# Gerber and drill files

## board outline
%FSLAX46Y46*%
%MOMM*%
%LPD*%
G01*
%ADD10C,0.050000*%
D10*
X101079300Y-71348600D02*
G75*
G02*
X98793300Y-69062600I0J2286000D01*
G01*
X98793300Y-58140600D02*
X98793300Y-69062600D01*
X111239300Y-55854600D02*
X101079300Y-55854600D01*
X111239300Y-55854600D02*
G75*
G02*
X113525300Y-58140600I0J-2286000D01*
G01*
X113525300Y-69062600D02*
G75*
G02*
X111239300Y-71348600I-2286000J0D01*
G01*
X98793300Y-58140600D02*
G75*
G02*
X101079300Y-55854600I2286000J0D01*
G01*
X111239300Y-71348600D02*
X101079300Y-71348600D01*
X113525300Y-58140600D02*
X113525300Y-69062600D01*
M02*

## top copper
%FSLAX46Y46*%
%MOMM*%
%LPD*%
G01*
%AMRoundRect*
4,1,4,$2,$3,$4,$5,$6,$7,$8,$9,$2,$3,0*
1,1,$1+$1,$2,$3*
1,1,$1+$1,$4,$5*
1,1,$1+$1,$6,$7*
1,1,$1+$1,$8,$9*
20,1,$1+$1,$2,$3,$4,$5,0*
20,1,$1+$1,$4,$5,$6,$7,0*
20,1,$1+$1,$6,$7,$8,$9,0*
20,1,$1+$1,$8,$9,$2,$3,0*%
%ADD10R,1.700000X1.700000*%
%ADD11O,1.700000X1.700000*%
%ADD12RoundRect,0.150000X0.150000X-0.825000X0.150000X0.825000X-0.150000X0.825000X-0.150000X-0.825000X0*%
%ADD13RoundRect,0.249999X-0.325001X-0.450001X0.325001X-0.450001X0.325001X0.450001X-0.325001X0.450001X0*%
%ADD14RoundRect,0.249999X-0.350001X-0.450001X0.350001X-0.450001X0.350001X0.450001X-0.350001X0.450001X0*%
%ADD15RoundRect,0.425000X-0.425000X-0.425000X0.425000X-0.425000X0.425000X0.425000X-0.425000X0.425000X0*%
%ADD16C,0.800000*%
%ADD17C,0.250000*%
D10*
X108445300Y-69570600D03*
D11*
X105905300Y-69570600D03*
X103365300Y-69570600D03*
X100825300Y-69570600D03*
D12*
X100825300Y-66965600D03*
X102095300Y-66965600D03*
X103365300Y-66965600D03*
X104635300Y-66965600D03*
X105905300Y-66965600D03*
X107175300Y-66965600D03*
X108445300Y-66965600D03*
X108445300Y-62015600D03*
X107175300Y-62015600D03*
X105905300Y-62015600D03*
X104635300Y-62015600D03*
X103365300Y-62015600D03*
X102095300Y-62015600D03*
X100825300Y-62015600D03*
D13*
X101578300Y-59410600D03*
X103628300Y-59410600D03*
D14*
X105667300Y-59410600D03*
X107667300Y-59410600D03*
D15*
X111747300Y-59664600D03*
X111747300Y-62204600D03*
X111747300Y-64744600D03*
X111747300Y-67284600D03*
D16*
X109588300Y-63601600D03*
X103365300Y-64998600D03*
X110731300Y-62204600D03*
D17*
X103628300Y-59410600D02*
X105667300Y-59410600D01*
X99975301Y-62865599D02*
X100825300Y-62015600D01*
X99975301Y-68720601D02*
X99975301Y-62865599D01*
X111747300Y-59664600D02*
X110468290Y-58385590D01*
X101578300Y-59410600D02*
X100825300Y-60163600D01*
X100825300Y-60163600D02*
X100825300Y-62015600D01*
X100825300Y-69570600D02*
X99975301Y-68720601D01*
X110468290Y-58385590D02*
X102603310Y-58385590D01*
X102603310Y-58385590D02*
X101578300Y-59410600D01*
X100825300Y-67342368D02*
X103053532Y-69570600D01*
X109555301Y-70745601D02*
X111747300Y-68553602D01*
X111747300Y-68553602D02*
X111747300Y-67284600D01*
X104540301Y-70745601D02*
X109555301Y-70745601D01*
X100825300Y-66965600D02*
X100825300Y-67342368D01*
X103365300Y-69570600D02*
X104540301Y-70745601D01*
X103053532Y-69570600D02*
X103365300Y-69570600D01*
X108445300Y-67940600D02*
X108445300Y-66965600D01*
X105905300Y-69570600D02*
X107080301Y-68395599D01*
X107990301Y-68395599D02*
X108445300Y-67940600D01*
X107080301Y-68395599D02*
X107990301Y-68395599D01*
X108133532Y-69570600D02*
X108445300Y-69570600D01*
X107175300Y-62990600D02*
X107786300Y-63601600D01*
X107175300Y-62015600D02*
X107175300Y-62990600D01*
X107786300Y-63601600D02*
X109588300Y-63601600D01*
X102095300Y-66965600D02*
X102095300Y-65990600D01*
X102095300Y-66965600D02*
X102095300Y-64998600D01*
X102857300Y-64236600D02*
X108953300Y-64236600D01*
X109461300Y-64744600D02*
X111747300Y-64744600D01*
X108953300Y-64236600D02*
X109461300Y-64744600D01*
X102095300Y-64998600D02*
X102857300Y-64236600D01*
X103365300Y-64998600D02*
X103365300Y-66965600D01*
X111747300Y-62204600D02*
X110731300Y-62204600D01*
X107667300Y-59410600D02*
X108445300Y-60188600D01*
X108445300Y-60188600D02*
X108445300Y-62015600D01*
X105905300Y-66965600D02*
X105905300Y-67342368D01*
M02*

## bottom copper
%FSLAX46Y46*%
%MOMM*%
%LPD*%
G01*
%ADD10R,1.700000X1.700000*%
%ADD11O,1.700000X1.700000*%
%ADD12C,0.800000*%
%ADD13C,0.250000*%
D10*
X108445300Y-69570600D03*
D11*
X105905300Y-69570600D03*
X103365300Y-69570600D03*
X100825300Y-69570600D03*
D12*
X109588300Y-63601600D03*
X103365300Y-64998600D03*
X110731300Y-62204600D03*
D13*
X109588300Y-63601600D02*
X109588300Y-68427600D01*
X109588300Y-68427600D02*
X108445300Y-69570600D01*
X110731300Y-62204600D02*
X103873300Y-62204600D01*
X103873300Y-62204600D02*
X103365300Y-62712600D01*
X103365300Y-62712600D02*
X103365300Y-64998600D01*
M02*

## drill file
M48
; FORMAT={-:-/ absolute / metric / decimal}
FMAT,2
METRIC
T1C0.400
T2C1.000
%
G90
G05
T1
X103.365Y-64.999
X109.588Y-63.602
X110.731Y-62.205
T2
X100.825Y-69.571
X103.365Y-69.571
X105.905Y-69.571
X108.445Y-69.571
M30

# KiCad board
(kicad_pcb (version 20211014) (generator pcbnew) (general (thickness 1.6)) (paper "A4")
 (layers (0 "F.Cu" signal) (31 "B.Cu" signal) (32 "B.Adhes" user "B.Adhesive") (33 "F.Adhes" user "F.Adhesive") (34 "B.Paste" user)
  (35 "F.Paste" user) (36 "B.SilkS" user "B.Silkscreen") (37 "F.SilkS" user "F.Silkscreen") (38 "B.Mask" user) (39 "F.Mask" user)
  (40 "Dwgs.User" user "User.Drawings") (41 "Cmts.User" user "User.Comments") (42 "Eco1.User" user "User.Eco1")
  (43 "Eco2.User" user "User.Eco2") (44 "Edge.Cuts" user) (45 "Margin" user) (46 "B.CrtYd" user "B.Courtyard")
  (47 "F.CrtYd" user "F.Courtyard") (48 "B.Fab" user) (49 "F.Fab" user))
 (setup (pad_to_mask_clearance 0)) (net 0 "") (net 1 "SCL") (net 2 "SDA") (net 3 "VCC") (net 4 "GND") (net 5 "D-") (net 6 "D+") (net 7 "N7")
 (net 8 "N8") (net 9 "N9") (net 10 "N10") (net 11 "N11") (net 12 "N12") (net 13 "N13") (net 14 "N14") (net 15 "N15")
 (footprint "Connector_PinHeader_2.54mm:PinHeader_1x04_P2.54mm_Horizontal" (layer "F.Cu") (at 108.4453 69.5706 -90)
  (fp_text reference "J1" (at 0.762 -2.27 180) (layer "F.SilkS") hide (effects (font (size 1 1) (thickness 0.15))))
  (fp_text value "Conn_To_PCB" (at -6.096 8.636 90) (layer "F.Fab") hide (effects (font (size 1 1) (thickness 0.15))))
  (pad "1" thru_hole rect locked (at 0 0 270) (size 1.7 1.7) (drill 1) (layers *.Cu *.Mask) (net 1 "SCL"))
  (pad "2" thru_hole oval locked (at 0 2.54 270) (size 1.7 1.7) (drill 1) (layers *.Cu *.Mask) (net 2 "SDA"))
  (pad "3" thru_hole oval locked (at 0 5.08 270) (size 1.7 1.7) (drill 1) (layers *.Cu *.Mask) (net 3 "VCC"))
  (pad "4" thru_hole oval locked (at 0 7.62 270) (size 1.7 1.7) (drill 1) (layers *.Cu *.Mask) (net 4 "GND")))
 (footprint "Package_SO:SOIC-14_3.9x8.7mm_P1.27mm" (layer "F.Cu") (at 104.6353 64.4906 90)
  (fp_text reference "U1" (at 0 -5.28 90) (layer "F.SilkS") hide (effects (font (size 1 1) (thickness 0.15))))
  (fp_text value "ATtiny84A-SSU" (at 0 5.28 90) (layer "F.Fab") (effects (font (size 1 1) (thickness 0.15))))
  (pad "1" smd roundrect locked (at -2.475 -3.81 90) (size 1.95 0.6) (layers "F.Cu" "F.Paste" "F.Mask") (roundrect_rratio 0.25)
   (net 3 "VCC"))
  (pad "2" smd roundrect locked (at -2.475 -2.54 90) (size 1.95 0.6) (layers "F.Cu" "F.Paste" "F.Mask") (roundrect_rratio 0.25) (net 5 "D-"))
  (pad "3" smd roundrect locked (at -2.475 -1.27 90) (size 1.95 0.6) (layers "F.Cu" "F.Paste" "F.Mask") (roundrect_rratio 0.25) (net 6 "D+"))
  (pad "4" smd roundrect locked (at -2.475 0 90) (size 1.95 0.6) (layers "F.Cu" "F.Paste" "F.Mask") (roundrect_rratio 0.25) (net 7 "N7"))
  (pad "5" smd roundrect locked (at -2.475 1.27 90) (size 1.95 0.6) (layers "F.Cu" "F.Paste" "F.Mask") (roundrect_rratio 0.25) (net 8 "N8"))
  (pad "6" smd roundrect locked (at -2.475 2.54 90) (size 1.95 0.6) (layers "F.Cu" "F.Paste" "F.Mask") (roundrect_rratio 0.25) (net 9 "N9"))
  (pad "7" smd roundrect locked (at -2.475 3.81 90) (size 1.95 0.6) (layers "F.Cu" "F.Paste" "F.Mask") (roundrect_rratio 0.25) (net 2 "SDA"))
  (pad "8" smd roundrect locked (at 2.475 3.81 90) (size 1.95 0.6) (layers "F.Cu" "F.Paste" "F.Mask") (roundrect_rratio 0.25) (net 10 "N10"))
  (pad "9" smd roundrect locked (at 2.475 2.54 90) (size 1.95 0.6) (layers "F.Cu" "F.Paste" "F.Mask") (roundrect_rratio 0.25) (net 1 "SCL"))
  (pad "10" smd roundrect locked (at 2.475 1.27 90) (size 1.95 0.6) (layers "F.Cu" "F.Paste" "F.Mask") (roundrect_rratio 0.25)
   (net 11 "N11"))
  (pad "11" smd roundrect locked (at 2.475 0 90) (size 1.95 0.6) (layers "F.Cu" "F.Paste" "F.Mask") (roundrect_rratio 0.25) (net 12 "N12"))
  (pad "12" smd roundrect locked (at 2.475 -1.27 90) (size 1.95 0.6) (layers "F.Cu" "F.Paste" "F.Mask") (roundrect_rratio 0.25)
   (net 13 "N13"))
  (pad "13" smd roundrect locked (at 2.475 -2.54 90) (size 1.95 0.6) (layers "F.Cu" "F.Paste" "F.Mask") (roundrect_rratio 0.25)
   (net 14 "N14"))
  (pad "14" smd roundrect locked (at 2.475 -3.81 90) (size 1.95 0.6) (layers "F.Cu" "F.Paste" "F.Mask") (roundrect_rratio 0.25)
   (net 4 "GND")))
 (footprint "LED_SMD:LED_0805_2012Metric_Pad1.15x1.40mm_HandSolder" (layer "F.Cu") (at 102.6033 59.4106)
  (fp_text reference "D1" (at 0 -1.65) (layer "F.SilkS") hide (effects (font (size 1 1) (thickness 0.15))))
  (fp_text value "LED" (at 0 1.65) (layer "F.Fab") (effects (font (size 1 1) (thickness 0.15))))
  (pad "1" smd roundrect locked (at -1.025 0) (size 1.15 1.4) (layers "F.Cu" "F.Paste" "F.Mask") (roundrect_rratio 0.2173904348)
   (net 4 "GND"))
  (pad "2" smd roundrect locked (at 1.025 0) (size 1.15 1.4) (layers "F.Cu" "F.Paste" "F.Mask") (roundrect_rratio 0.2173904348)
   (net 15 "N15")))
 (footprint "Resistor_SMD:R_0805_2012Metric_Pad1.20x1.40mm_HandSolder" (layer "F.Cu") (at 106.6673 59.4106)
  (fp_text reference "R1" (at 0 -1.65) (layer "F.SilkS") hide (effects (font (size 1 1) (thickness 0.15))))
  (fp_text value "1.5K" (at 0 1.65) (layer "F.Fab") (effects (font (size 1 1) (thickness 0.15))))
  (pad "1" smd roundrect locked (at -1 0) (size 1.2 1.4) (layers "F.Cu" "F.Paste" "F.Mask") (roundrect_rratio 0.2083325) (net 15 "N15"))
  (pad "2" smd roundrect locked (at 1 0) (size 1.2 1.4) (layers "F.Cu" "F.Paste" "F.Mask") (roundrect_rratio 0.2083325) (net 10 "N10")))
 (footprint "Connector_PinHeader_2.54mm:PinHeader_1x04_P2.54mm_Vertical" (layer "F.Cu") (at 111.7473 59.6646)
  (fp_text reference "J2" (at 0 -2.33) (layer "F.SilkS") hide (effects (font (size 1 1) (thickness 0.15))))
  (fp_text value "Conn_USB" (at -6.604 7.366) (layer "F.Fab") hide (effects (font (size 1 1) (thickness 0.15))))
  (pad "1" smd roundrect locked (at 0 0) (size 1.7 1.7) (layers "F.Cu" "F.Paste" "F.Mask") (roundrect_rratio 0.25) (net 4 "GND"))
  (pad "2" smd roundrect locked (at 0 2.54) (size 1.7 1.7) (layers "F.Cu" "F.Paste" "F.Mask") (roundrect_rratio 0.25) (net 6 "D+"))
  (pad "3" smd roundrect locked (at 0 5.08) (size 1.7 1.7) (layers "F.Cu" "F.Paste" "F.Mask") (roundrect_rratio 0.25) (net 5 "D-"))
  (pad "4" smd roundrect locked (at 0 7.62) (size 1.7 1.7) (layers "F.Cu" "F.Paste" "F.Mask") (roundrect_rratio 0.25) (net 3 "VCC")))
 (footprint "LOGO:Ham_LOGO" (layer "B.Cu") (at 108.6993 61.6966 180)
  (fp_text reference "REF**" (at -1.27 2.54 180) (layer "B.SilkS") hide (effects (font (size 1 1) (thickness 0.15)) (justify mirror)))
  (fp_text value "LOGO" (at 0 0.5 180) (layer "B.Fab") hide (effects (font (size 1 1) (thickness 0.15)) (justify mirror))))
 (gr_arc (start 101.0793 71.3486) (mid 99.462854 70.679046) (end 98.7933 69.0626) (layer "Edge.Cuts") (width 0.05))
 (gr_line (start 98.7933 58.1406) (end 98.7933 69.0626) (layer "Edge.Cuts") (width 0.05))
 (gr_line (start 111.2393 55.8546) (end 101.0793 55.8546) (layer "Edge.Cuts") (width 0.05))
 (gr_arc (start 111.2393 55.8546) (mid 112.855746 56.524154) (end 113.5253 58.1406) (layer "Edge.Cuts") (width 0.05))
 (gr_arc (start 113.5253 69.0626) (mid 112.855746 70.679046) (end 111.2393 71.3486) (layer "Edge.Cuts") (width 0.05))
 (gr_arc (start 98.7933 58.1406) (mid 99.462854 56.524154) (end 101.0793 55.8546) (layer "Edge.Cuts") (width 0.05))
 (gr_line (start 111.2393 71.3486) (end 101.0793 71.3486) (layer "Edge.Cuts") (width 0.05))
 (gr_line (start 113.5253 58.1406) (end 113.5253 69.0626) (layer "Edge.Cuts") (width 0.05))
 (segment (start 103.6283 59.4106) (end 105.6673 59.4106) (width 0.25) (layer "F.Cu") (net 15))
 (segment (start 99.975301 62.865599) (end 100.8253 62.0156) (width 0.25) (layer "F.Cu") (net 4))
 (segment (start 99.975301 68.720601) (end 99.975301 62.865599) (width 0.25) (layer "F.Cu") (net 4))
 (segment (start 111.7473 59.6646) (end 110.46829 58.38559) (width 0.25) (layer "F.Cu") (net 4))
 (segment (start 101.5783 59.4106) (end 100.8253 60.1636) (width 0.25) (layer "F.Cu") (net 4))
 (segment (start 100.8253 60.1636) (end 100.8253 62.0156) (width 0.25) (layer "F.Cu") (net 4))
 (segment (start 100.8253 69.5706) (end 99.975301 68.720601) (width 0.25) (layer "F.Cu") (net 4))
 (segment (start 110.46829 58.38559) (end 102.60331 58.38559) (width 0.25) (layer "F.Cu") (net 4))
 (segment (start 102.60331 58.38559) (end 101.5783 59.4106) (width 0.25) (layer "F.Cu") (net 4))
 (segment (start 100.8253 67.342368) (end 103.053532 69.5706) (width 0.25) (layer "F.Cu") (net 3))
 (segment (start 109.555301 70.745601) (end 111.7473 68.553602) (width 0.25) (layer "F.Cu") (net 3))
 (segment (start 111.7473 68.553602) (end 111.7473 67.2846) (width 0.25) (layer "F.Cu") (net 3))
 (segment (start 104.540301 70.745601) (end 109.555301 70.745601) (width 0.25) (layer "F.Cu") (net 3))
 (segment (start 100.8253 66.9656) (end 100.8253 67.342368) (width 0.25) (layer "F.Cu") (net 3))
 (segment (start 103.3653 69.5706) (end 104.540301 70.745601) (width 0.25) (layer "F.Cu") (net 3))
 (segment (start 103.053532 69.5706) (end 103.3653 69.5706) (width 0.25) (layer "F.Cu") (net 3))
 (segment (start 108.4453 67.9406) (end 108.4453 66.9656) (width 0.25) (layer "F.Cu") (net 2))
 (segment (start 105.9053 69.5706) (end 107.080301 68.395599) (width 0.25) (layer "F.Cu") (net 2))
 (segment (start 107.990301 68.395599) (end 108.4453 67.9406) (width 0.25) (layer "F.Cu") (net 2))
 (segment (start 107.080301 68.395599) (end 107.990301 68.395599) (width 0.25) (layer "F.Cu") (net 2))
 (segment (start 108.133532 69.5706) (end 108.4453 69.5706) (width 0.25) (layer "F.Cu") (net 1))
 (segment (start 107.1753 62.9906) (end 107.7863 63.6016) (width 0.25) (layer "F.Cu") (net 1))
 (segment (start 107.1753 62.0156) (end 107.1753 62.9906) (width 0.25) (layer "F.Cu") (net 1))
 (segment (start 107.7863 63.6016) (end 109.5883 63.6016) (width 0.25) (layer "F.Cu") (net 1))
 (via (at 109.5883 63.6016) (size 0.8) (drill 0.4) (layers "F.Cu" "B.Cu") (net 1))
 (segment (start 109.5883 63.6016) (end 109.5883 68.4276) (width 0.25) (layer "B.Cu") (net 1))
 (segment (start 109.5883 68.4276) (end 108.4453 69.5706) (width 0.25) (layer "B.Cu") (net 1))
 (segment (start 102.0953 66.9656) (end 102.0953 65.9906) (width 0.25) (layer "F.Cu") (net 5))
 (segment (start 102.0953 66.9656) (end 102.0953 64.9986) (width 0.25) (layer "F.Cu") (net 5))
 (segment (start 102.8573 64.2366) (end 108.9533 64.2366) (width 0.25) (layer "F.Cu") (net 5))
 (segment (start 109.4613 64.7446) (end 111.7473 64.7446) (width 0.25) (layer "F.Cu") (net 5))
 (segment (start 108.9533 64.2366) (end 109.4613 64.7446) (width 0.25) (layer "F.Cu") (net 5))
 (segment (start 102.0953 64.9986) (end 102.8573 64.2366) (width 0.25) (layer "F.Cu") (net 5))
 (segment (start 103.3653 64.9986) (end 103.3653 66.9656) (width 0.25) (layer "F.Cu") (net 6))
 (segment (start 111.7473 62.2046) (end 110.7313 62.2046) (width 0.25) (layer "F.Cu") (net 6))
 (via (at 103.3653 64.9986) (size 0.8) (drill 0.4) (layers "F.Cu" "B.Cu") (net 6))
 (via (at 110.7313 62.2046) (size 0.8) (drill 0.4) (layers "F.Cu" "B.Cu") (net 6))
 (segment (start 110.7313 62.2046) (end 103.8733 62.2046) (width 0.25) (layer "B.Cu") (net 6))
 (segment (start 103.8733 62.2046) (end 103.3653 62.7126) (width 0.25) (layer "B.Cu") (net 6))
 (segment (start 103.3653 62.7126) (end 103.3653 64.9986) (width 0.25) (layer "B.Cu") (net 6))
 (segment (start 107.6673 59.4106) (end 108.4453 60.1886) (width 0.25) (layer "F.Cu") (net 10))
 (segment (start 108.4453 60.1886) (end 108.4453 62.0156) (width 0.25) (layer "F.Cu") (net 10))
 (segment (start 105.9053 66.9656) (end 105.9053 67.342368) (width 0.25) (layer "F.Cu") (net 8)))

